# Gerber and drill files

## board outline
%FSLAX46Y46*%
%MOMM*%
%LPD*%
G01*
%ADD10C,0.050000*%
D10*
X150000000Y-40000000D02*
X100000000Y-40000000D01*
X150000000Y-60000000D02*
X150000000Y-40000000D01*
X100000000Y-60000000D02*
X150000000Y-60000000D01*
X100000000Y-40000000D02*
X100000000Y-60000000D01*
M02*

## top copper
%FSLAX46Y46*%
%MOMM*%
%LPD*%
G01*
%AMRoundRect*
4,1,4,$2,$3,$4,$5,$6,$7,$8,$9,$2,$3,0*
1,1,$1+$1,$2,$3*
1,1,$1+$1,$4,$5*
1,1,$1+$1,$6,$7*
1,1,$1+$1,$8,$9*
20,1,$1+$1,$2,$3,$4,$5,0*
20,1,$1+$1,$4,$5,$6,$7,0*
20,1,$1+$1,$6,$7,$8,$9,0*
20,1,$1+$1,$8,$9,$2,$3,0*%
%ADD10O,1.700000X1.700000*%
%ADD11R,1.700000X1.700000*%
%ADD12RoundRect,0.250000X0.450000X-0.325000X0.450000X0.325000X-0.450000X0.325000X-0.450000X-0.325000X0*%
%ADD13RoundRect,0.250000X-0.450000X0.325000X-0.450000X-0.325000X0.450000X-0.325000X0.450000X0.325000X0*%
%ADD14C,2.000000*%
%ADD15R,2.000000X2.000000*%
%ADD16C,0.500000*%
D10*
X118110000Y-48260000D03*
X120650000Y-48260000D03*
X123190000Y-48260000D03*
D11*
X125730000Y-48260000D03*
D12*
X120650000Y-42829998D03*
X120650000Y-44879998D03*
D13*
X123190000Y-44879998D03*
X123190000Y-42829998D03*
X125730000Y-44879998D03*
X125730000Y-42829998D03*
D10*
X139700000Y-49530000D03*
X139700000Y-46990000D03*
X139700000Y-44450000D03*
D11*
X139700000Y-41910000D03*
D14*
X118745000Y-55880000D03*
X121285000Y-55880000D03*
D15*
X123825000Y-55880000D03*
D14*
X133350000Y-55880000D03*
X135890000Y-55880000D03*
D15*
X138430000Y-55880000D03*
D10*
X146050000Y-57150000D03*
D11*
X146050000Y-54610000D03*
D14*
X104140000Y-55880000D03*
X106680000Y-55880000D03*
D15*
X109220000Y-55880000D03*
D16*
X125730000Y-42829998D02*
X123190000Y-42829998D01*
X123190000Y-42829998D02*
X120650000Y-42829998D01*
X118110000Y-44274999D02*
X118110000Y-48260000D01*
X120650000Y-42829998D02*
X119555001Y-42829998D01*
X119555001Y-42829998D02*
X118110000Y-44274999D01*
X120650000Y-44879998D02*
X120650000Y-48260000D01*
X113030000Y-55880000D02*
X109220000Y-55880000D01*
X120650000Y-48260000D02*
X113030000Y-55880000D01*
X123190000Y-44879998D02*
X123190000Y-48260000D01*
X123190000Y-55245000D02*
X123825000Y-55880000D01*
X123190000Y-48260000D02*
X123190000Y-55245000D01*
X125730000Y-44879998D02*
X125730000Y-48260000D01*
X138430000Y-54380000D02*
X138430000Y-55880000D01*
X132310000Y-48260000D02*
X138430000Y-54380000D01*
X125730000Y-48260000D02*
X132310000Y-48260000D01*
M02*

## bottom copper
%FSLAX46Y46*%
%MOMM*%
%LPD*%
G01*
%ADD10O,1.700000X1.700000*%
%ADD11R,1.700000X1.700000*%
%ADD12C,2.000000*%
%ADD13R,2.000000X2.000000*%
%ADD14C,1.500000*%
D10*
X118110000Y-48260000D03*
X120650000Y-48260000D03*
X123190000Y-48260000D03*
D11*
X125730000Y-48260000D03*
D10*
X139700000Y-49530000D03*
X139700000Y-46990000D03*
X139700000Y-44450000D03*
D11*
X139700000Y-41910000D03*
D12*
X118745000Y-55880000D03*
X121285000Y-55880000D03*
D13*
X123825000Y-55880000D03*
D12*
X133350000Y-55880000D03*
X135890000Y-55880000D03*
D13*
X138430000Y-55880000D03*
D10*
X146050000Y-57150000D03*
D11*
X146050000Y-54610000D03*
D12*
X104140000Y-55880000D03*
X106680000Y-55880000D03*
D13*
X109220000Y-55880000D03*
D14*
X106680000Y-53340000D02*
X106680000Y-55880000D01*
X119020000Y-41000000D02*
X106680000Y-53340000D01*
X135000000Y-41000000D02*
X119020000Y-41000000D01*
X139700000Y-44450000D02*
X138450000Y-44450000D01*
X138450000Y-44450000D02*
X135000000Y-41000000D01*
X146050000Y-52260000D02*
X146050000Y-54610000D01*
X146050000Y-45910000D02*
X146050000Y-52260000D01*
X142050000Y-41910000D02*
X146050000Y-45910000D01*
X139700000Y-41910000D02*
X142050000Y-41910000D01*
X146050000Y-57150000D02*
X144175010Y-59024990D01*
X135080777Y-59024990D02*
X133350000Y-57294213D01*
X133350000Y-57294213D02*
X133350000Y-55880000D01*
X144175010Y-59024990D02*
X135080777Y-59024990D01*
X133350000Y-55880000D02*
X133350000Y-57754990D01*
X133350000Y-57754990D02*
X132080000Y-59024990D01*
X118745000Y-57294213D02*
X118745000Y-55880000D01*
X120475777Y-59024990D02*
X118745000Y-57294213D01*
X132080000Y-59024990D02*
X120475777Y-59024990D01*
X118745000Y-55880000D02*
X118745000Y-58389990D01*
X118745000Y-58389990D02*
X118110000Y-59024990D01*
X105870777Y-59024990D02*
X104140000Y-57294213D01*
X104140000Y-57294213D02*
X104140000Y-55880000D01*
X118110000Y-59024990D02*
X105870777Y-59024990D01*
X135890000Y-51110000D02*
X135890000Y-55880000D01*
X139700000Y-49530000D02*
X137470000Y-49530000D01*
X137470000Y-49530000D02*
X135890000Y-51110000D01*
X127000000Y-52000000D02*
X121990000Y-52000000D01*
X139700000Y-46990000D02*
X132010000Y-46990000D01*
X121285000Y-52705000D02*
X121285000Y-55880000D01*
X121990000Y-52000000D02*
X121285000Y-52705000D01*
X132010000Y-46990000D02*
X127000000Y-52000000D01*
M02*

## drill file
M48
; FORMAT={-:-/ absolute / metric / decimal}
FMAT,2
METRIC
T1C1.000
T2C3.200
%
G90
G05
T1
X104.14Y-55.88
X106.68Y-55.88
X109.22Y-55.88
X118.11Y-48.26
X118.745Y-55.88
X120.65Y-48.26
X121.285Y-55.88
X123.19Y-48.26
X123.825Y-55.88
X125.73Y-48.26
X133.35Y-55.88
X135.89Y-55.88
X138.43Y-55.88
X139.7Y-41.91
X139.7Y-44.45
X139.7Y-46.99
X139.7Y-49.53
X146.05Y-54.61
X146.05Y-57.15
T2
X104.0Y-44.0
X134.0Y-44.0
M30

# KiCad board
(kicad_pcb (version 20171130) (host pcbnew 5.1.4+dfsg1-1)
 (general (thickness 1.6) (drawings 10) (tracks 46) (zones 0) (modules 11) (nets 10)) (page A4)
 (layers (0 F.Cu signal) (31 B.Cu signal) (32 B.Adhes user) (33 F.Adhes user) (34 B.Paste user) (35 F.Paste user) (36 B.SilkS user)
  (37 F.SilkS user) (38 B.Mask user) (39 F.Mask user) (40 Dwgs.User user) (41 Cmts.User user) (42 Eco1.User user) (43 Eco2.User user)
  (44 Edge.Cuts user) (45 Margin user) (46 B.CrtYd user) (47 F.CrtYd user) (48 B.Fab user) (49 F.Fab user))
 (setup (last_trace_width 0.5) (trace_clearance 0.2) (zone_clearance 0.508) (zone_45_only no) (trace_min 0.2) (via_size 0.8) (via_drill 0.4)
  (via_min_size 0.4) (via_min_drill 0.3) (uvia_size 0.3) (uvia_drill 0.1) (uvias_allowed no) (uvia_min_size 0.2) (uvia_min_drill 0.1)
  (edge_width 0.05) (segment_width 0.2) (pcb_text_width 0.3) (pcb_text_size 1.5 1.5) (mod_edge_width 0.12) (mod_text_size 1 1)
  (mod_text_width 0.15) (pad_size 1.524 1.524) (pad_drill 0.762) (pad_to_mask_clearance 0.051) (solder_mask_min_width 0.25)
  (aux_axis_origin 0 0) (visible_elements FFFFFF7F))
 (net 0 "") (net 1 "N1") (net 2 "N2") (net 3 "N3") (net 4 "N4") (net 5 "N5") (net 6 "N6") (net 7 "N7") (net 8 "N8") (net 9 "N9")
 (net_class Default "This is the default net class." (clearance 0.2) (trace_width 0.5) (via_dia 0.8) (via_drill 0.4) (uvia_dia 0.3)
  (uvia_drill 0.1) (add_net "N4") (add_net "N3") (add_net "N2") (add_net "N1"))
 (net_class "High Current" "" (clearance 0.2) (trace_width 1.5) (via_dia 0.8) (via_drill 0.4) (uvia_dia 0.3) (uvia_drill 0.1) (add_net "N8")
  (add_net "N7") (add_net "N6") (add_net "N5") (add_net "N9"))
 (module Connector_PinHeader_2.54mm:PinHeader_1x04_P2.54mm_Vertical (layer F.Cu) (at 125.73 48.26 270)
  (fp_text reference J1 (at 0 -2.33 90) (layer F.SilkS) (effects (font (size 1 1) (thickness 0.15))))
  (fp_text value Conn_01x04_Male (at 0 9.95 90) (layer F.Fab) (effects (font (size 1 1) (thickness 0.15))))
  (pad 4 thru_hole oval (at 0 7.62 270) (size 1.7 1.7) (drill 1) (layers *.Cu *.Mask) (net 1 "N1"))
  (pad 3 thru_hole oval (at 0 5.08 270) (size 1.7 1.7) (drill 1) (layers *.Cu *.Mask) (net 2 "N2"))
  (pad 2 thru_hole oval (at 0 2.54 270) (size 1.7 1.7) (drill 1) (layers *.Cu *.Mask) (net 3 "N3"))
  (pad 1 thru_hole rect (at 0 0 270) (size 1.7 1.7) (drill 1) (layers *.Cu *.Mask) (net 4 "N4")))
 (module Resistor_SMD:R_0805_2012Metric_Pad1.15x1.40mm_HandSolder (layer F.Cu) (at 120.65 43.854998 90)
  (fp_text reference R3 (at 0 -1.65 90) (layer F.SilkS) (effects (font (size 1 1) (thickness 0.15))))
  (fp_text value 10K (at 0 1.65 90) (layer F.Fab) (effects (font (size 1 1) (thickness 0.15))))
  (pad 2 smd roundrect (at 1.025 0 90) (size 1.15 1.4) (layers F.Cu F.Paste F.Mask) (roundrect_rratio 0.217391) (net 1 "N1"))
  (pad 1 smd roundrect (at -1.025 0 90) (size 1.15 1.4) (layers F.Cu F.Paste F.Mask) (roundrect_rratio 0.217391) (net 2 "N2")))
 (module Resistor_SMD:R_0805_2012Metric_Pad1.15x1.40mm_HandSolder (layer F.Cu) (at 123.19 43.854998 270)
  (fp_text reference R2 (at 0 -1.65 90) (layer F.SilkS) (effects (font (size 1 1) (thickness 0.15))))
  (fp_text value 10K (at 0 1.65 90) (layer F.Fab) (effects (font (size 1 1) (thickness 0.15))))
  (pad 2 smd roundrect (at 1.025 0 270) (size 1.15 1.4) (layers F.Cu F.Paste F.Mask) (roundrect_rratio 0.217391) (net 3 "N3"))
  (pad 1 smd roundrect (at -1.025 0 270) (size 1.15 1.4) (layers F.Cu F.Paste F.Mask) (roundrect_rratio 0.217391) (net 1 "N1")))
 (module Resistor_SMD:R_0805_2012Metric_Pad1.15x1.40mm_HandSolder (layer F.Cu) (at 125.73 43.854998 270)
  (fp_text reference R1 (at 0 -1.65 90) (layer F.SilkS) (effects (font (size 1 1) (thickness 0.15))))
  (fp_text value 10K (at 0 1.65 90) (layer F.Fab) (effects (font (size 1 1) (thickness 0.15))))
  (pad 2 smd roundrect (at 1.025 0 270) (size 1.15 1.4) (layers F.Cu F.Paste F.Mask) (roundrect_rratio 0.217391) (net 4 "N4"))
  (pad 1 smd roundrect (at -1.025 0 270) (size 1.15 1.4) (layers F.Cu F.Paste F.Mask) (roundrect_rratio 0.217391) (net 1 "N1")))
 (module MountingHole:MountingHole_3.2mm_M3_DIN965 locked (layer F.Cu) (at 134 44)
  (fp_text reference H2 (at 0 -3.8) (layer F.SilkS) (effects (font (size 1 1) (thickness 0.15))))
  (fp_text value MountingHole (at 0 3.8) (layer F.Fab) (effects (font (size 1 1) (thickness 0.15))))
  (pad 1 np_thru_hole circle (at 0 0) (size 3.2 3.2) (drill 3.2) (layers *.Cu *.Mask)))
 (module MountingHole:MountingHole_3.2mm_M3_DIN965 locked (layer F.Cu) (at 104 44)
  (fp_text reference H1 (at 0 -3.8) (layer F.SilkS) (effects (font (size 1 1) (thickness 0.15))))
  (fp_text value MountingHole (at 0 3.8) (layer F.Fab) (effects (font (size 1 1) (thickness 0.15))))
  (pad 1 np_thru_hole circle (at 0 0) (size 3.2 3.2) (drill 3.2) (layers *.Cu *.Mask)))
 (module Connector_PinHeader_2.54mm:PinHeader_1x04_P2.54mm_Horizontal (layer F.Cu) (at 139.7 41.91)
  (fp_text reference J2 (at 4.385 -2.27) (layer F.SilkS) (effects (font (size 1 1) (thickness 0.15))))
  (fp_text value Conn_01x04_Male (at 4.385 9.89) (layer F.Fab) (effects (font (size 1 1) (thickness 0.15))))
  (pad 4 thru_hole oval (at 0 7.62) (size 1.7 1.7) (drill 1) (layers *.Cu *.Mask) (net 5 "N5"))
  (pad 3 thru_hole oval (at 0 5.08) (size 1.7 1.7) (drill 1) (layers *.Cu *.Mask) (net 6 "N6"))
  (pad 2 thru_hole oval (at 0 2.54) (size 1.7 1.7) (drill 1) (layers *.Cu *.Mask) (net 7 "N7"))
  (pad 1 thru_hole rect (at 0 0) (size 1.7 1.7) (drill 1) (layers *.Cu *.Mask) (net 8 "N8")))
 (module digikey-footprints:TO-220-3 (layer F.Cu) (at 123.825 55.88 180)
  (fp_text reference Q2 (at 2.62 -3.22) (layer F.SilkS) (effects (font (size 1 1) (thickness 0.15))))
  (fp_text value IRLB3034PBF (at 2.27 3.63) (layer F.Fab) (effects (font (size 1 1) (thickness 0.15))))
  (pad 3 thru_hole circle (at 5.08 0 180) (size 2 2) (drill 1) (layers *.Cu *.Mask) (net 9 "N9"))
  (pad 2 thru_hole circle (at 2.54 0 180) (size 2 2) (drill 1) (layers *.Cu *.Mask) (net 6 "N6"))
  (pad 1 thru_hole rect (at 0 0 180) (size 2 2) (drill 1) (layers *.Cu *.Mask) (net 3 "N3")))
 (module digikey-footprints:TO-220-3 (layer F.Cu) (at 138.43 55.88 180)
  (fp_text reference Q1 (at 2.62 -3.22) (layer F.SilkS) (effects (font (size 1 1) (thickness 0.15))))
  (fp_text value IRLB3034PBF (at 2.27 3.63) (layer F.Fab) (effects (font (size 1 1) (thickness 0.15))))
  (pad 3 thru_hole circle (at 5.08 0 180) (size 2 2) (drill 1) (layers *.Cu *.Mask) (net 9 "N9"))
  (pad 2 thru_hole circle (at 2.54 0 180) (size 2 2) (drill 1) (layers *.Cu *.Mask) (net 5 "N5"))
  (pad 1 thru_hole rect (at 0 0 180) (size 2 2) (drill 1) (layers *.Cu *.Mask) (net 4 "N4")))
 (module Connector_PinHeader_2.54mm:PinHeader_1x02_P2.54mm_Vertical (layer F.Cu) (at 146.05 54.61)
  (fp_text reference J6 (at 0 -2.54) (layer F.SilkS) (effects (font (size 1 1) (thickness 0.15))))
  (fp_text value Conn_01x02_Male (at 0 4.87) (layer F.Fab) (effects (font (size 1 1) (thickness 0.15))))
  (pad 2 thru_hole oval (at 0 2.54) (size 1.7 1.7) (drill 1) (layers *.Cu *.Mask) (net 9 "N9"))
  (pad 1 thru_hole rect (at 0 0) (size 1.7 1.7) (drill 1) (layers *.Cu *.Mask) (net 8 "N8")))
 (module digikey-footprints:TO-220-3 (layer F.Cu) (at 109.22 55.88 180)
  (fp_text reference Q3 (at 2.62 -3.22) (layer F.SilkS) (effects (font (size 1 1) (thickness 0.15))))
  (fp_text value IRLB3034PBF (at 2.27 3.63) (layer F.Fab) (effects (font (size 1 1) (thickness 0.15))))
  (pad 3 thru_hole circle (at 5.08 0 180) (size 2 2) (drill 1) (layers *.Cu *.Mask) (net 9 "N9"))
  (pad 2 thru_hole circle (at 2.54 0 180) (size 2 2) (drill 1) (layers *.Cu *.Mask) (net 7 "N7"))
  (pad 1 thru_hole rect (at 0 0 180) (size 2 2) (drill 1) (layers *.Cu *.Mask) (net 2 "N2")))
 (gr_line (start 150 40) (end 100 40) (layer Edge.Cuts) (width 0.05))
 (gr_line (start 150 60) (end 150 40) (layer Edge.Cuts) (width 0.05))
 (gr_line (start 100 60) (end 150 60) (layer Edge.Cuts) (width 0.05))
 (gr_line (start 100 40) (end 100 60) (layer Edge.Cuts) (width 0.05))
 (segment (start 125.73 42.829998) (end 123.19 42.829998) (width 0.5) (layer F.Cu) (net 1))
 (segment (start 123.19 42.829998) (end 120.65 42.829998) (width 0.5) (layer F.Cu) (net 1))
 (segment (start 118.11 44.274999) (end 118.11 48.26) (width 0.5) (layer F.Cu) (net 1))
 (segment (start 120.65 42.829998) (end 119.555001 42.829998) (width 0.5) (layer F.Cu) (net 1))
 (segment (start 119.555001 42.829998) (end 118.11 44.274999) (width 0.5) (layer F.Cu) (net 1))
 (segment (start 120.65 44.879998) (end 120.65 48.26) (width 0.5) (layer F.Cu) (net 2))
 (segment (start 113.03 55.88) (end 109.22 55.88) (width 0.5) (layer F.Cu) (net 2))
 (segment (start 120.65 48.26) (end 113.03 55.88) (width 0.5) (layer F.Cu) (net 2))
 (segment (start 123.19 44.879998) (end 123.19 48.26) (width 0.5) (layer F.Cu) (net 3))
 (segment (start 123.19 55.245) (end 123.825 55.88) (width 0.5) (layer F.Cu) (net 3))
 (segment (start 123.19 48.26) (end 123.19 55.245) (width 0.5) (layer F.Cu) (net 3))
 (segment (start 125.73 44.879998) (end 125.73 48.26) (width 0.5) (layer F.Cu) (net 4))
 (segment (start 138.43 54.38) (end 138.43 55.88) (width 0.5) (layer F.Cu) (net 4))
 (segment (start 132.31 48.26) (end 138.43 54.38) (width 0.5) (layer F.Cu) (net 4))
 (segment (start 125.73 48.26) (end 132.31 48.26) (width 0.5) (layer F.Cu) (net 4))
 (segment (start 106.68 53.34) (end 106.68 55.88) (width 1.5) (layer B.Cu) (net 7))
 (segment (start 119.02 41) (end 106.68 53.34) (width 1.5) (layer B.Cu) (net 7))
 (segment (start 135 41) (end 119.02 41) (width 1.5) (layer B.Cu) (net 7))
 (segment (start 139.7 44.45) (end 138.45 44.45) (width 1.5) (layer B.Cu) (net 7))
 (segment (start 138.45 44.45) (end 135 41) (width 1.5) (layer B.Cu) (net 7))
 (segment (start 146.05 52.26) (end 146.05 54.61) (width 1.5) (layer B.Cu) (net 8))
 (segment (start 146.05 45.91) (end 146.05 52.26) (width 1.5) (layer B.Cu) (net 8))
 (segment (start 142.05 41.91) (end 146.05 45.91) (width 1.5) (layer B.Cu) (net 8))
 (segment (start 139.7 41.91) (end 142.05 41.91) (width 1.5) (layer B.Cu) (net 8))
 (segment (start 146.05 57.15) (end 144.17501 59.02499) (width 1.5) (layer B.Cu) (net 9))
 (segment (start 135.080777 59.02499) (end 133.35 57.294213) (width 1.5) (layer B.Cu) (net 9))
 (segment (start 133.35 57.294213) (end 133.35 55.88) (width 1.5) (layer B.Cu) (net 9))
 (segment (start 144.17501 59.02499) (end 135.080777 59.02499) (width 1.5) (layer B.Cu) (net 9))
 (segment (start 133.35 55.88) (end 133.35 57.75499) (width 1.5) (layer B.Cu) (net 9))
 (segment (start 133.35 57.75499) (end 132.08 59.02499) (width 1.5) (layer B.Cu) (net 9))
 (segment (start 118.745 57.294213) (end 118.745 55.88) (width 1.5) (layer B.Cu) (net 9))
 (segment (start 120.475777 59.02499) (end 118.745 57.294213) (width 1.5) (layer B.Cu) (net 9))
 (segment (start 132.08 59.02499) (end 120.475777 59.02499) (width 1.5) (layer B.Cu) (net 9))
 (segment (start 118.745 55.88) (end 118.745 58.38999) (width 1.5) (layer B.Cu) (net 9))
 (segment (start 118.745 58.38999) (end 118.11 59.02499) (width 1.5) (layer B.Cu) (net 9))
 (segment (start 105.870777 59.02499) (end 104.14 57.294213) (width 1.5) (layer B.Cu) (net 9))
 (segment (start 104.14 57.294213) (end 104.14 55.88) (width 1.5) (layer B.Cu) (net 9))
 (segment (start 118.11 59.02499) (end 105.870777 59.02499) (width 1.5) (layer B.Cu) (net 9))
 (segment (start 135.89 51.11) (end 135.89 55.88) (width 1.5) (layer B.Cu) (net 5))
 (segment (start 139.7 49.53) (end 137.47 49.53) (width 1.5) (layer B.Cu) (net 5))
 (segment (start 137.47 49.53) (end 135.89 51.11) (width 1.5) (layer B.Cu) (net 5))
 (segment (start 127 52) (end 121.99 52) (width 1.5) (layer B.Cu) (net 6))
 (segment (start 139.7 46.99) (end 132.01 46.99) (width 1.5) (layer B.Cu) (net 6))
 (segment (start 121.285 52.705) (end 121.285 55.88) (width 1.5) (layer B.Cu) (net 6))
 (segment (start 121.99 52) (end 121.285 52.705) (width 1.5) (layer B.Cu) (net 6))
 (segment (start 132.01 46.99) (end 127 52) (width 1.5) (layer B.Cu) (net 6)))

